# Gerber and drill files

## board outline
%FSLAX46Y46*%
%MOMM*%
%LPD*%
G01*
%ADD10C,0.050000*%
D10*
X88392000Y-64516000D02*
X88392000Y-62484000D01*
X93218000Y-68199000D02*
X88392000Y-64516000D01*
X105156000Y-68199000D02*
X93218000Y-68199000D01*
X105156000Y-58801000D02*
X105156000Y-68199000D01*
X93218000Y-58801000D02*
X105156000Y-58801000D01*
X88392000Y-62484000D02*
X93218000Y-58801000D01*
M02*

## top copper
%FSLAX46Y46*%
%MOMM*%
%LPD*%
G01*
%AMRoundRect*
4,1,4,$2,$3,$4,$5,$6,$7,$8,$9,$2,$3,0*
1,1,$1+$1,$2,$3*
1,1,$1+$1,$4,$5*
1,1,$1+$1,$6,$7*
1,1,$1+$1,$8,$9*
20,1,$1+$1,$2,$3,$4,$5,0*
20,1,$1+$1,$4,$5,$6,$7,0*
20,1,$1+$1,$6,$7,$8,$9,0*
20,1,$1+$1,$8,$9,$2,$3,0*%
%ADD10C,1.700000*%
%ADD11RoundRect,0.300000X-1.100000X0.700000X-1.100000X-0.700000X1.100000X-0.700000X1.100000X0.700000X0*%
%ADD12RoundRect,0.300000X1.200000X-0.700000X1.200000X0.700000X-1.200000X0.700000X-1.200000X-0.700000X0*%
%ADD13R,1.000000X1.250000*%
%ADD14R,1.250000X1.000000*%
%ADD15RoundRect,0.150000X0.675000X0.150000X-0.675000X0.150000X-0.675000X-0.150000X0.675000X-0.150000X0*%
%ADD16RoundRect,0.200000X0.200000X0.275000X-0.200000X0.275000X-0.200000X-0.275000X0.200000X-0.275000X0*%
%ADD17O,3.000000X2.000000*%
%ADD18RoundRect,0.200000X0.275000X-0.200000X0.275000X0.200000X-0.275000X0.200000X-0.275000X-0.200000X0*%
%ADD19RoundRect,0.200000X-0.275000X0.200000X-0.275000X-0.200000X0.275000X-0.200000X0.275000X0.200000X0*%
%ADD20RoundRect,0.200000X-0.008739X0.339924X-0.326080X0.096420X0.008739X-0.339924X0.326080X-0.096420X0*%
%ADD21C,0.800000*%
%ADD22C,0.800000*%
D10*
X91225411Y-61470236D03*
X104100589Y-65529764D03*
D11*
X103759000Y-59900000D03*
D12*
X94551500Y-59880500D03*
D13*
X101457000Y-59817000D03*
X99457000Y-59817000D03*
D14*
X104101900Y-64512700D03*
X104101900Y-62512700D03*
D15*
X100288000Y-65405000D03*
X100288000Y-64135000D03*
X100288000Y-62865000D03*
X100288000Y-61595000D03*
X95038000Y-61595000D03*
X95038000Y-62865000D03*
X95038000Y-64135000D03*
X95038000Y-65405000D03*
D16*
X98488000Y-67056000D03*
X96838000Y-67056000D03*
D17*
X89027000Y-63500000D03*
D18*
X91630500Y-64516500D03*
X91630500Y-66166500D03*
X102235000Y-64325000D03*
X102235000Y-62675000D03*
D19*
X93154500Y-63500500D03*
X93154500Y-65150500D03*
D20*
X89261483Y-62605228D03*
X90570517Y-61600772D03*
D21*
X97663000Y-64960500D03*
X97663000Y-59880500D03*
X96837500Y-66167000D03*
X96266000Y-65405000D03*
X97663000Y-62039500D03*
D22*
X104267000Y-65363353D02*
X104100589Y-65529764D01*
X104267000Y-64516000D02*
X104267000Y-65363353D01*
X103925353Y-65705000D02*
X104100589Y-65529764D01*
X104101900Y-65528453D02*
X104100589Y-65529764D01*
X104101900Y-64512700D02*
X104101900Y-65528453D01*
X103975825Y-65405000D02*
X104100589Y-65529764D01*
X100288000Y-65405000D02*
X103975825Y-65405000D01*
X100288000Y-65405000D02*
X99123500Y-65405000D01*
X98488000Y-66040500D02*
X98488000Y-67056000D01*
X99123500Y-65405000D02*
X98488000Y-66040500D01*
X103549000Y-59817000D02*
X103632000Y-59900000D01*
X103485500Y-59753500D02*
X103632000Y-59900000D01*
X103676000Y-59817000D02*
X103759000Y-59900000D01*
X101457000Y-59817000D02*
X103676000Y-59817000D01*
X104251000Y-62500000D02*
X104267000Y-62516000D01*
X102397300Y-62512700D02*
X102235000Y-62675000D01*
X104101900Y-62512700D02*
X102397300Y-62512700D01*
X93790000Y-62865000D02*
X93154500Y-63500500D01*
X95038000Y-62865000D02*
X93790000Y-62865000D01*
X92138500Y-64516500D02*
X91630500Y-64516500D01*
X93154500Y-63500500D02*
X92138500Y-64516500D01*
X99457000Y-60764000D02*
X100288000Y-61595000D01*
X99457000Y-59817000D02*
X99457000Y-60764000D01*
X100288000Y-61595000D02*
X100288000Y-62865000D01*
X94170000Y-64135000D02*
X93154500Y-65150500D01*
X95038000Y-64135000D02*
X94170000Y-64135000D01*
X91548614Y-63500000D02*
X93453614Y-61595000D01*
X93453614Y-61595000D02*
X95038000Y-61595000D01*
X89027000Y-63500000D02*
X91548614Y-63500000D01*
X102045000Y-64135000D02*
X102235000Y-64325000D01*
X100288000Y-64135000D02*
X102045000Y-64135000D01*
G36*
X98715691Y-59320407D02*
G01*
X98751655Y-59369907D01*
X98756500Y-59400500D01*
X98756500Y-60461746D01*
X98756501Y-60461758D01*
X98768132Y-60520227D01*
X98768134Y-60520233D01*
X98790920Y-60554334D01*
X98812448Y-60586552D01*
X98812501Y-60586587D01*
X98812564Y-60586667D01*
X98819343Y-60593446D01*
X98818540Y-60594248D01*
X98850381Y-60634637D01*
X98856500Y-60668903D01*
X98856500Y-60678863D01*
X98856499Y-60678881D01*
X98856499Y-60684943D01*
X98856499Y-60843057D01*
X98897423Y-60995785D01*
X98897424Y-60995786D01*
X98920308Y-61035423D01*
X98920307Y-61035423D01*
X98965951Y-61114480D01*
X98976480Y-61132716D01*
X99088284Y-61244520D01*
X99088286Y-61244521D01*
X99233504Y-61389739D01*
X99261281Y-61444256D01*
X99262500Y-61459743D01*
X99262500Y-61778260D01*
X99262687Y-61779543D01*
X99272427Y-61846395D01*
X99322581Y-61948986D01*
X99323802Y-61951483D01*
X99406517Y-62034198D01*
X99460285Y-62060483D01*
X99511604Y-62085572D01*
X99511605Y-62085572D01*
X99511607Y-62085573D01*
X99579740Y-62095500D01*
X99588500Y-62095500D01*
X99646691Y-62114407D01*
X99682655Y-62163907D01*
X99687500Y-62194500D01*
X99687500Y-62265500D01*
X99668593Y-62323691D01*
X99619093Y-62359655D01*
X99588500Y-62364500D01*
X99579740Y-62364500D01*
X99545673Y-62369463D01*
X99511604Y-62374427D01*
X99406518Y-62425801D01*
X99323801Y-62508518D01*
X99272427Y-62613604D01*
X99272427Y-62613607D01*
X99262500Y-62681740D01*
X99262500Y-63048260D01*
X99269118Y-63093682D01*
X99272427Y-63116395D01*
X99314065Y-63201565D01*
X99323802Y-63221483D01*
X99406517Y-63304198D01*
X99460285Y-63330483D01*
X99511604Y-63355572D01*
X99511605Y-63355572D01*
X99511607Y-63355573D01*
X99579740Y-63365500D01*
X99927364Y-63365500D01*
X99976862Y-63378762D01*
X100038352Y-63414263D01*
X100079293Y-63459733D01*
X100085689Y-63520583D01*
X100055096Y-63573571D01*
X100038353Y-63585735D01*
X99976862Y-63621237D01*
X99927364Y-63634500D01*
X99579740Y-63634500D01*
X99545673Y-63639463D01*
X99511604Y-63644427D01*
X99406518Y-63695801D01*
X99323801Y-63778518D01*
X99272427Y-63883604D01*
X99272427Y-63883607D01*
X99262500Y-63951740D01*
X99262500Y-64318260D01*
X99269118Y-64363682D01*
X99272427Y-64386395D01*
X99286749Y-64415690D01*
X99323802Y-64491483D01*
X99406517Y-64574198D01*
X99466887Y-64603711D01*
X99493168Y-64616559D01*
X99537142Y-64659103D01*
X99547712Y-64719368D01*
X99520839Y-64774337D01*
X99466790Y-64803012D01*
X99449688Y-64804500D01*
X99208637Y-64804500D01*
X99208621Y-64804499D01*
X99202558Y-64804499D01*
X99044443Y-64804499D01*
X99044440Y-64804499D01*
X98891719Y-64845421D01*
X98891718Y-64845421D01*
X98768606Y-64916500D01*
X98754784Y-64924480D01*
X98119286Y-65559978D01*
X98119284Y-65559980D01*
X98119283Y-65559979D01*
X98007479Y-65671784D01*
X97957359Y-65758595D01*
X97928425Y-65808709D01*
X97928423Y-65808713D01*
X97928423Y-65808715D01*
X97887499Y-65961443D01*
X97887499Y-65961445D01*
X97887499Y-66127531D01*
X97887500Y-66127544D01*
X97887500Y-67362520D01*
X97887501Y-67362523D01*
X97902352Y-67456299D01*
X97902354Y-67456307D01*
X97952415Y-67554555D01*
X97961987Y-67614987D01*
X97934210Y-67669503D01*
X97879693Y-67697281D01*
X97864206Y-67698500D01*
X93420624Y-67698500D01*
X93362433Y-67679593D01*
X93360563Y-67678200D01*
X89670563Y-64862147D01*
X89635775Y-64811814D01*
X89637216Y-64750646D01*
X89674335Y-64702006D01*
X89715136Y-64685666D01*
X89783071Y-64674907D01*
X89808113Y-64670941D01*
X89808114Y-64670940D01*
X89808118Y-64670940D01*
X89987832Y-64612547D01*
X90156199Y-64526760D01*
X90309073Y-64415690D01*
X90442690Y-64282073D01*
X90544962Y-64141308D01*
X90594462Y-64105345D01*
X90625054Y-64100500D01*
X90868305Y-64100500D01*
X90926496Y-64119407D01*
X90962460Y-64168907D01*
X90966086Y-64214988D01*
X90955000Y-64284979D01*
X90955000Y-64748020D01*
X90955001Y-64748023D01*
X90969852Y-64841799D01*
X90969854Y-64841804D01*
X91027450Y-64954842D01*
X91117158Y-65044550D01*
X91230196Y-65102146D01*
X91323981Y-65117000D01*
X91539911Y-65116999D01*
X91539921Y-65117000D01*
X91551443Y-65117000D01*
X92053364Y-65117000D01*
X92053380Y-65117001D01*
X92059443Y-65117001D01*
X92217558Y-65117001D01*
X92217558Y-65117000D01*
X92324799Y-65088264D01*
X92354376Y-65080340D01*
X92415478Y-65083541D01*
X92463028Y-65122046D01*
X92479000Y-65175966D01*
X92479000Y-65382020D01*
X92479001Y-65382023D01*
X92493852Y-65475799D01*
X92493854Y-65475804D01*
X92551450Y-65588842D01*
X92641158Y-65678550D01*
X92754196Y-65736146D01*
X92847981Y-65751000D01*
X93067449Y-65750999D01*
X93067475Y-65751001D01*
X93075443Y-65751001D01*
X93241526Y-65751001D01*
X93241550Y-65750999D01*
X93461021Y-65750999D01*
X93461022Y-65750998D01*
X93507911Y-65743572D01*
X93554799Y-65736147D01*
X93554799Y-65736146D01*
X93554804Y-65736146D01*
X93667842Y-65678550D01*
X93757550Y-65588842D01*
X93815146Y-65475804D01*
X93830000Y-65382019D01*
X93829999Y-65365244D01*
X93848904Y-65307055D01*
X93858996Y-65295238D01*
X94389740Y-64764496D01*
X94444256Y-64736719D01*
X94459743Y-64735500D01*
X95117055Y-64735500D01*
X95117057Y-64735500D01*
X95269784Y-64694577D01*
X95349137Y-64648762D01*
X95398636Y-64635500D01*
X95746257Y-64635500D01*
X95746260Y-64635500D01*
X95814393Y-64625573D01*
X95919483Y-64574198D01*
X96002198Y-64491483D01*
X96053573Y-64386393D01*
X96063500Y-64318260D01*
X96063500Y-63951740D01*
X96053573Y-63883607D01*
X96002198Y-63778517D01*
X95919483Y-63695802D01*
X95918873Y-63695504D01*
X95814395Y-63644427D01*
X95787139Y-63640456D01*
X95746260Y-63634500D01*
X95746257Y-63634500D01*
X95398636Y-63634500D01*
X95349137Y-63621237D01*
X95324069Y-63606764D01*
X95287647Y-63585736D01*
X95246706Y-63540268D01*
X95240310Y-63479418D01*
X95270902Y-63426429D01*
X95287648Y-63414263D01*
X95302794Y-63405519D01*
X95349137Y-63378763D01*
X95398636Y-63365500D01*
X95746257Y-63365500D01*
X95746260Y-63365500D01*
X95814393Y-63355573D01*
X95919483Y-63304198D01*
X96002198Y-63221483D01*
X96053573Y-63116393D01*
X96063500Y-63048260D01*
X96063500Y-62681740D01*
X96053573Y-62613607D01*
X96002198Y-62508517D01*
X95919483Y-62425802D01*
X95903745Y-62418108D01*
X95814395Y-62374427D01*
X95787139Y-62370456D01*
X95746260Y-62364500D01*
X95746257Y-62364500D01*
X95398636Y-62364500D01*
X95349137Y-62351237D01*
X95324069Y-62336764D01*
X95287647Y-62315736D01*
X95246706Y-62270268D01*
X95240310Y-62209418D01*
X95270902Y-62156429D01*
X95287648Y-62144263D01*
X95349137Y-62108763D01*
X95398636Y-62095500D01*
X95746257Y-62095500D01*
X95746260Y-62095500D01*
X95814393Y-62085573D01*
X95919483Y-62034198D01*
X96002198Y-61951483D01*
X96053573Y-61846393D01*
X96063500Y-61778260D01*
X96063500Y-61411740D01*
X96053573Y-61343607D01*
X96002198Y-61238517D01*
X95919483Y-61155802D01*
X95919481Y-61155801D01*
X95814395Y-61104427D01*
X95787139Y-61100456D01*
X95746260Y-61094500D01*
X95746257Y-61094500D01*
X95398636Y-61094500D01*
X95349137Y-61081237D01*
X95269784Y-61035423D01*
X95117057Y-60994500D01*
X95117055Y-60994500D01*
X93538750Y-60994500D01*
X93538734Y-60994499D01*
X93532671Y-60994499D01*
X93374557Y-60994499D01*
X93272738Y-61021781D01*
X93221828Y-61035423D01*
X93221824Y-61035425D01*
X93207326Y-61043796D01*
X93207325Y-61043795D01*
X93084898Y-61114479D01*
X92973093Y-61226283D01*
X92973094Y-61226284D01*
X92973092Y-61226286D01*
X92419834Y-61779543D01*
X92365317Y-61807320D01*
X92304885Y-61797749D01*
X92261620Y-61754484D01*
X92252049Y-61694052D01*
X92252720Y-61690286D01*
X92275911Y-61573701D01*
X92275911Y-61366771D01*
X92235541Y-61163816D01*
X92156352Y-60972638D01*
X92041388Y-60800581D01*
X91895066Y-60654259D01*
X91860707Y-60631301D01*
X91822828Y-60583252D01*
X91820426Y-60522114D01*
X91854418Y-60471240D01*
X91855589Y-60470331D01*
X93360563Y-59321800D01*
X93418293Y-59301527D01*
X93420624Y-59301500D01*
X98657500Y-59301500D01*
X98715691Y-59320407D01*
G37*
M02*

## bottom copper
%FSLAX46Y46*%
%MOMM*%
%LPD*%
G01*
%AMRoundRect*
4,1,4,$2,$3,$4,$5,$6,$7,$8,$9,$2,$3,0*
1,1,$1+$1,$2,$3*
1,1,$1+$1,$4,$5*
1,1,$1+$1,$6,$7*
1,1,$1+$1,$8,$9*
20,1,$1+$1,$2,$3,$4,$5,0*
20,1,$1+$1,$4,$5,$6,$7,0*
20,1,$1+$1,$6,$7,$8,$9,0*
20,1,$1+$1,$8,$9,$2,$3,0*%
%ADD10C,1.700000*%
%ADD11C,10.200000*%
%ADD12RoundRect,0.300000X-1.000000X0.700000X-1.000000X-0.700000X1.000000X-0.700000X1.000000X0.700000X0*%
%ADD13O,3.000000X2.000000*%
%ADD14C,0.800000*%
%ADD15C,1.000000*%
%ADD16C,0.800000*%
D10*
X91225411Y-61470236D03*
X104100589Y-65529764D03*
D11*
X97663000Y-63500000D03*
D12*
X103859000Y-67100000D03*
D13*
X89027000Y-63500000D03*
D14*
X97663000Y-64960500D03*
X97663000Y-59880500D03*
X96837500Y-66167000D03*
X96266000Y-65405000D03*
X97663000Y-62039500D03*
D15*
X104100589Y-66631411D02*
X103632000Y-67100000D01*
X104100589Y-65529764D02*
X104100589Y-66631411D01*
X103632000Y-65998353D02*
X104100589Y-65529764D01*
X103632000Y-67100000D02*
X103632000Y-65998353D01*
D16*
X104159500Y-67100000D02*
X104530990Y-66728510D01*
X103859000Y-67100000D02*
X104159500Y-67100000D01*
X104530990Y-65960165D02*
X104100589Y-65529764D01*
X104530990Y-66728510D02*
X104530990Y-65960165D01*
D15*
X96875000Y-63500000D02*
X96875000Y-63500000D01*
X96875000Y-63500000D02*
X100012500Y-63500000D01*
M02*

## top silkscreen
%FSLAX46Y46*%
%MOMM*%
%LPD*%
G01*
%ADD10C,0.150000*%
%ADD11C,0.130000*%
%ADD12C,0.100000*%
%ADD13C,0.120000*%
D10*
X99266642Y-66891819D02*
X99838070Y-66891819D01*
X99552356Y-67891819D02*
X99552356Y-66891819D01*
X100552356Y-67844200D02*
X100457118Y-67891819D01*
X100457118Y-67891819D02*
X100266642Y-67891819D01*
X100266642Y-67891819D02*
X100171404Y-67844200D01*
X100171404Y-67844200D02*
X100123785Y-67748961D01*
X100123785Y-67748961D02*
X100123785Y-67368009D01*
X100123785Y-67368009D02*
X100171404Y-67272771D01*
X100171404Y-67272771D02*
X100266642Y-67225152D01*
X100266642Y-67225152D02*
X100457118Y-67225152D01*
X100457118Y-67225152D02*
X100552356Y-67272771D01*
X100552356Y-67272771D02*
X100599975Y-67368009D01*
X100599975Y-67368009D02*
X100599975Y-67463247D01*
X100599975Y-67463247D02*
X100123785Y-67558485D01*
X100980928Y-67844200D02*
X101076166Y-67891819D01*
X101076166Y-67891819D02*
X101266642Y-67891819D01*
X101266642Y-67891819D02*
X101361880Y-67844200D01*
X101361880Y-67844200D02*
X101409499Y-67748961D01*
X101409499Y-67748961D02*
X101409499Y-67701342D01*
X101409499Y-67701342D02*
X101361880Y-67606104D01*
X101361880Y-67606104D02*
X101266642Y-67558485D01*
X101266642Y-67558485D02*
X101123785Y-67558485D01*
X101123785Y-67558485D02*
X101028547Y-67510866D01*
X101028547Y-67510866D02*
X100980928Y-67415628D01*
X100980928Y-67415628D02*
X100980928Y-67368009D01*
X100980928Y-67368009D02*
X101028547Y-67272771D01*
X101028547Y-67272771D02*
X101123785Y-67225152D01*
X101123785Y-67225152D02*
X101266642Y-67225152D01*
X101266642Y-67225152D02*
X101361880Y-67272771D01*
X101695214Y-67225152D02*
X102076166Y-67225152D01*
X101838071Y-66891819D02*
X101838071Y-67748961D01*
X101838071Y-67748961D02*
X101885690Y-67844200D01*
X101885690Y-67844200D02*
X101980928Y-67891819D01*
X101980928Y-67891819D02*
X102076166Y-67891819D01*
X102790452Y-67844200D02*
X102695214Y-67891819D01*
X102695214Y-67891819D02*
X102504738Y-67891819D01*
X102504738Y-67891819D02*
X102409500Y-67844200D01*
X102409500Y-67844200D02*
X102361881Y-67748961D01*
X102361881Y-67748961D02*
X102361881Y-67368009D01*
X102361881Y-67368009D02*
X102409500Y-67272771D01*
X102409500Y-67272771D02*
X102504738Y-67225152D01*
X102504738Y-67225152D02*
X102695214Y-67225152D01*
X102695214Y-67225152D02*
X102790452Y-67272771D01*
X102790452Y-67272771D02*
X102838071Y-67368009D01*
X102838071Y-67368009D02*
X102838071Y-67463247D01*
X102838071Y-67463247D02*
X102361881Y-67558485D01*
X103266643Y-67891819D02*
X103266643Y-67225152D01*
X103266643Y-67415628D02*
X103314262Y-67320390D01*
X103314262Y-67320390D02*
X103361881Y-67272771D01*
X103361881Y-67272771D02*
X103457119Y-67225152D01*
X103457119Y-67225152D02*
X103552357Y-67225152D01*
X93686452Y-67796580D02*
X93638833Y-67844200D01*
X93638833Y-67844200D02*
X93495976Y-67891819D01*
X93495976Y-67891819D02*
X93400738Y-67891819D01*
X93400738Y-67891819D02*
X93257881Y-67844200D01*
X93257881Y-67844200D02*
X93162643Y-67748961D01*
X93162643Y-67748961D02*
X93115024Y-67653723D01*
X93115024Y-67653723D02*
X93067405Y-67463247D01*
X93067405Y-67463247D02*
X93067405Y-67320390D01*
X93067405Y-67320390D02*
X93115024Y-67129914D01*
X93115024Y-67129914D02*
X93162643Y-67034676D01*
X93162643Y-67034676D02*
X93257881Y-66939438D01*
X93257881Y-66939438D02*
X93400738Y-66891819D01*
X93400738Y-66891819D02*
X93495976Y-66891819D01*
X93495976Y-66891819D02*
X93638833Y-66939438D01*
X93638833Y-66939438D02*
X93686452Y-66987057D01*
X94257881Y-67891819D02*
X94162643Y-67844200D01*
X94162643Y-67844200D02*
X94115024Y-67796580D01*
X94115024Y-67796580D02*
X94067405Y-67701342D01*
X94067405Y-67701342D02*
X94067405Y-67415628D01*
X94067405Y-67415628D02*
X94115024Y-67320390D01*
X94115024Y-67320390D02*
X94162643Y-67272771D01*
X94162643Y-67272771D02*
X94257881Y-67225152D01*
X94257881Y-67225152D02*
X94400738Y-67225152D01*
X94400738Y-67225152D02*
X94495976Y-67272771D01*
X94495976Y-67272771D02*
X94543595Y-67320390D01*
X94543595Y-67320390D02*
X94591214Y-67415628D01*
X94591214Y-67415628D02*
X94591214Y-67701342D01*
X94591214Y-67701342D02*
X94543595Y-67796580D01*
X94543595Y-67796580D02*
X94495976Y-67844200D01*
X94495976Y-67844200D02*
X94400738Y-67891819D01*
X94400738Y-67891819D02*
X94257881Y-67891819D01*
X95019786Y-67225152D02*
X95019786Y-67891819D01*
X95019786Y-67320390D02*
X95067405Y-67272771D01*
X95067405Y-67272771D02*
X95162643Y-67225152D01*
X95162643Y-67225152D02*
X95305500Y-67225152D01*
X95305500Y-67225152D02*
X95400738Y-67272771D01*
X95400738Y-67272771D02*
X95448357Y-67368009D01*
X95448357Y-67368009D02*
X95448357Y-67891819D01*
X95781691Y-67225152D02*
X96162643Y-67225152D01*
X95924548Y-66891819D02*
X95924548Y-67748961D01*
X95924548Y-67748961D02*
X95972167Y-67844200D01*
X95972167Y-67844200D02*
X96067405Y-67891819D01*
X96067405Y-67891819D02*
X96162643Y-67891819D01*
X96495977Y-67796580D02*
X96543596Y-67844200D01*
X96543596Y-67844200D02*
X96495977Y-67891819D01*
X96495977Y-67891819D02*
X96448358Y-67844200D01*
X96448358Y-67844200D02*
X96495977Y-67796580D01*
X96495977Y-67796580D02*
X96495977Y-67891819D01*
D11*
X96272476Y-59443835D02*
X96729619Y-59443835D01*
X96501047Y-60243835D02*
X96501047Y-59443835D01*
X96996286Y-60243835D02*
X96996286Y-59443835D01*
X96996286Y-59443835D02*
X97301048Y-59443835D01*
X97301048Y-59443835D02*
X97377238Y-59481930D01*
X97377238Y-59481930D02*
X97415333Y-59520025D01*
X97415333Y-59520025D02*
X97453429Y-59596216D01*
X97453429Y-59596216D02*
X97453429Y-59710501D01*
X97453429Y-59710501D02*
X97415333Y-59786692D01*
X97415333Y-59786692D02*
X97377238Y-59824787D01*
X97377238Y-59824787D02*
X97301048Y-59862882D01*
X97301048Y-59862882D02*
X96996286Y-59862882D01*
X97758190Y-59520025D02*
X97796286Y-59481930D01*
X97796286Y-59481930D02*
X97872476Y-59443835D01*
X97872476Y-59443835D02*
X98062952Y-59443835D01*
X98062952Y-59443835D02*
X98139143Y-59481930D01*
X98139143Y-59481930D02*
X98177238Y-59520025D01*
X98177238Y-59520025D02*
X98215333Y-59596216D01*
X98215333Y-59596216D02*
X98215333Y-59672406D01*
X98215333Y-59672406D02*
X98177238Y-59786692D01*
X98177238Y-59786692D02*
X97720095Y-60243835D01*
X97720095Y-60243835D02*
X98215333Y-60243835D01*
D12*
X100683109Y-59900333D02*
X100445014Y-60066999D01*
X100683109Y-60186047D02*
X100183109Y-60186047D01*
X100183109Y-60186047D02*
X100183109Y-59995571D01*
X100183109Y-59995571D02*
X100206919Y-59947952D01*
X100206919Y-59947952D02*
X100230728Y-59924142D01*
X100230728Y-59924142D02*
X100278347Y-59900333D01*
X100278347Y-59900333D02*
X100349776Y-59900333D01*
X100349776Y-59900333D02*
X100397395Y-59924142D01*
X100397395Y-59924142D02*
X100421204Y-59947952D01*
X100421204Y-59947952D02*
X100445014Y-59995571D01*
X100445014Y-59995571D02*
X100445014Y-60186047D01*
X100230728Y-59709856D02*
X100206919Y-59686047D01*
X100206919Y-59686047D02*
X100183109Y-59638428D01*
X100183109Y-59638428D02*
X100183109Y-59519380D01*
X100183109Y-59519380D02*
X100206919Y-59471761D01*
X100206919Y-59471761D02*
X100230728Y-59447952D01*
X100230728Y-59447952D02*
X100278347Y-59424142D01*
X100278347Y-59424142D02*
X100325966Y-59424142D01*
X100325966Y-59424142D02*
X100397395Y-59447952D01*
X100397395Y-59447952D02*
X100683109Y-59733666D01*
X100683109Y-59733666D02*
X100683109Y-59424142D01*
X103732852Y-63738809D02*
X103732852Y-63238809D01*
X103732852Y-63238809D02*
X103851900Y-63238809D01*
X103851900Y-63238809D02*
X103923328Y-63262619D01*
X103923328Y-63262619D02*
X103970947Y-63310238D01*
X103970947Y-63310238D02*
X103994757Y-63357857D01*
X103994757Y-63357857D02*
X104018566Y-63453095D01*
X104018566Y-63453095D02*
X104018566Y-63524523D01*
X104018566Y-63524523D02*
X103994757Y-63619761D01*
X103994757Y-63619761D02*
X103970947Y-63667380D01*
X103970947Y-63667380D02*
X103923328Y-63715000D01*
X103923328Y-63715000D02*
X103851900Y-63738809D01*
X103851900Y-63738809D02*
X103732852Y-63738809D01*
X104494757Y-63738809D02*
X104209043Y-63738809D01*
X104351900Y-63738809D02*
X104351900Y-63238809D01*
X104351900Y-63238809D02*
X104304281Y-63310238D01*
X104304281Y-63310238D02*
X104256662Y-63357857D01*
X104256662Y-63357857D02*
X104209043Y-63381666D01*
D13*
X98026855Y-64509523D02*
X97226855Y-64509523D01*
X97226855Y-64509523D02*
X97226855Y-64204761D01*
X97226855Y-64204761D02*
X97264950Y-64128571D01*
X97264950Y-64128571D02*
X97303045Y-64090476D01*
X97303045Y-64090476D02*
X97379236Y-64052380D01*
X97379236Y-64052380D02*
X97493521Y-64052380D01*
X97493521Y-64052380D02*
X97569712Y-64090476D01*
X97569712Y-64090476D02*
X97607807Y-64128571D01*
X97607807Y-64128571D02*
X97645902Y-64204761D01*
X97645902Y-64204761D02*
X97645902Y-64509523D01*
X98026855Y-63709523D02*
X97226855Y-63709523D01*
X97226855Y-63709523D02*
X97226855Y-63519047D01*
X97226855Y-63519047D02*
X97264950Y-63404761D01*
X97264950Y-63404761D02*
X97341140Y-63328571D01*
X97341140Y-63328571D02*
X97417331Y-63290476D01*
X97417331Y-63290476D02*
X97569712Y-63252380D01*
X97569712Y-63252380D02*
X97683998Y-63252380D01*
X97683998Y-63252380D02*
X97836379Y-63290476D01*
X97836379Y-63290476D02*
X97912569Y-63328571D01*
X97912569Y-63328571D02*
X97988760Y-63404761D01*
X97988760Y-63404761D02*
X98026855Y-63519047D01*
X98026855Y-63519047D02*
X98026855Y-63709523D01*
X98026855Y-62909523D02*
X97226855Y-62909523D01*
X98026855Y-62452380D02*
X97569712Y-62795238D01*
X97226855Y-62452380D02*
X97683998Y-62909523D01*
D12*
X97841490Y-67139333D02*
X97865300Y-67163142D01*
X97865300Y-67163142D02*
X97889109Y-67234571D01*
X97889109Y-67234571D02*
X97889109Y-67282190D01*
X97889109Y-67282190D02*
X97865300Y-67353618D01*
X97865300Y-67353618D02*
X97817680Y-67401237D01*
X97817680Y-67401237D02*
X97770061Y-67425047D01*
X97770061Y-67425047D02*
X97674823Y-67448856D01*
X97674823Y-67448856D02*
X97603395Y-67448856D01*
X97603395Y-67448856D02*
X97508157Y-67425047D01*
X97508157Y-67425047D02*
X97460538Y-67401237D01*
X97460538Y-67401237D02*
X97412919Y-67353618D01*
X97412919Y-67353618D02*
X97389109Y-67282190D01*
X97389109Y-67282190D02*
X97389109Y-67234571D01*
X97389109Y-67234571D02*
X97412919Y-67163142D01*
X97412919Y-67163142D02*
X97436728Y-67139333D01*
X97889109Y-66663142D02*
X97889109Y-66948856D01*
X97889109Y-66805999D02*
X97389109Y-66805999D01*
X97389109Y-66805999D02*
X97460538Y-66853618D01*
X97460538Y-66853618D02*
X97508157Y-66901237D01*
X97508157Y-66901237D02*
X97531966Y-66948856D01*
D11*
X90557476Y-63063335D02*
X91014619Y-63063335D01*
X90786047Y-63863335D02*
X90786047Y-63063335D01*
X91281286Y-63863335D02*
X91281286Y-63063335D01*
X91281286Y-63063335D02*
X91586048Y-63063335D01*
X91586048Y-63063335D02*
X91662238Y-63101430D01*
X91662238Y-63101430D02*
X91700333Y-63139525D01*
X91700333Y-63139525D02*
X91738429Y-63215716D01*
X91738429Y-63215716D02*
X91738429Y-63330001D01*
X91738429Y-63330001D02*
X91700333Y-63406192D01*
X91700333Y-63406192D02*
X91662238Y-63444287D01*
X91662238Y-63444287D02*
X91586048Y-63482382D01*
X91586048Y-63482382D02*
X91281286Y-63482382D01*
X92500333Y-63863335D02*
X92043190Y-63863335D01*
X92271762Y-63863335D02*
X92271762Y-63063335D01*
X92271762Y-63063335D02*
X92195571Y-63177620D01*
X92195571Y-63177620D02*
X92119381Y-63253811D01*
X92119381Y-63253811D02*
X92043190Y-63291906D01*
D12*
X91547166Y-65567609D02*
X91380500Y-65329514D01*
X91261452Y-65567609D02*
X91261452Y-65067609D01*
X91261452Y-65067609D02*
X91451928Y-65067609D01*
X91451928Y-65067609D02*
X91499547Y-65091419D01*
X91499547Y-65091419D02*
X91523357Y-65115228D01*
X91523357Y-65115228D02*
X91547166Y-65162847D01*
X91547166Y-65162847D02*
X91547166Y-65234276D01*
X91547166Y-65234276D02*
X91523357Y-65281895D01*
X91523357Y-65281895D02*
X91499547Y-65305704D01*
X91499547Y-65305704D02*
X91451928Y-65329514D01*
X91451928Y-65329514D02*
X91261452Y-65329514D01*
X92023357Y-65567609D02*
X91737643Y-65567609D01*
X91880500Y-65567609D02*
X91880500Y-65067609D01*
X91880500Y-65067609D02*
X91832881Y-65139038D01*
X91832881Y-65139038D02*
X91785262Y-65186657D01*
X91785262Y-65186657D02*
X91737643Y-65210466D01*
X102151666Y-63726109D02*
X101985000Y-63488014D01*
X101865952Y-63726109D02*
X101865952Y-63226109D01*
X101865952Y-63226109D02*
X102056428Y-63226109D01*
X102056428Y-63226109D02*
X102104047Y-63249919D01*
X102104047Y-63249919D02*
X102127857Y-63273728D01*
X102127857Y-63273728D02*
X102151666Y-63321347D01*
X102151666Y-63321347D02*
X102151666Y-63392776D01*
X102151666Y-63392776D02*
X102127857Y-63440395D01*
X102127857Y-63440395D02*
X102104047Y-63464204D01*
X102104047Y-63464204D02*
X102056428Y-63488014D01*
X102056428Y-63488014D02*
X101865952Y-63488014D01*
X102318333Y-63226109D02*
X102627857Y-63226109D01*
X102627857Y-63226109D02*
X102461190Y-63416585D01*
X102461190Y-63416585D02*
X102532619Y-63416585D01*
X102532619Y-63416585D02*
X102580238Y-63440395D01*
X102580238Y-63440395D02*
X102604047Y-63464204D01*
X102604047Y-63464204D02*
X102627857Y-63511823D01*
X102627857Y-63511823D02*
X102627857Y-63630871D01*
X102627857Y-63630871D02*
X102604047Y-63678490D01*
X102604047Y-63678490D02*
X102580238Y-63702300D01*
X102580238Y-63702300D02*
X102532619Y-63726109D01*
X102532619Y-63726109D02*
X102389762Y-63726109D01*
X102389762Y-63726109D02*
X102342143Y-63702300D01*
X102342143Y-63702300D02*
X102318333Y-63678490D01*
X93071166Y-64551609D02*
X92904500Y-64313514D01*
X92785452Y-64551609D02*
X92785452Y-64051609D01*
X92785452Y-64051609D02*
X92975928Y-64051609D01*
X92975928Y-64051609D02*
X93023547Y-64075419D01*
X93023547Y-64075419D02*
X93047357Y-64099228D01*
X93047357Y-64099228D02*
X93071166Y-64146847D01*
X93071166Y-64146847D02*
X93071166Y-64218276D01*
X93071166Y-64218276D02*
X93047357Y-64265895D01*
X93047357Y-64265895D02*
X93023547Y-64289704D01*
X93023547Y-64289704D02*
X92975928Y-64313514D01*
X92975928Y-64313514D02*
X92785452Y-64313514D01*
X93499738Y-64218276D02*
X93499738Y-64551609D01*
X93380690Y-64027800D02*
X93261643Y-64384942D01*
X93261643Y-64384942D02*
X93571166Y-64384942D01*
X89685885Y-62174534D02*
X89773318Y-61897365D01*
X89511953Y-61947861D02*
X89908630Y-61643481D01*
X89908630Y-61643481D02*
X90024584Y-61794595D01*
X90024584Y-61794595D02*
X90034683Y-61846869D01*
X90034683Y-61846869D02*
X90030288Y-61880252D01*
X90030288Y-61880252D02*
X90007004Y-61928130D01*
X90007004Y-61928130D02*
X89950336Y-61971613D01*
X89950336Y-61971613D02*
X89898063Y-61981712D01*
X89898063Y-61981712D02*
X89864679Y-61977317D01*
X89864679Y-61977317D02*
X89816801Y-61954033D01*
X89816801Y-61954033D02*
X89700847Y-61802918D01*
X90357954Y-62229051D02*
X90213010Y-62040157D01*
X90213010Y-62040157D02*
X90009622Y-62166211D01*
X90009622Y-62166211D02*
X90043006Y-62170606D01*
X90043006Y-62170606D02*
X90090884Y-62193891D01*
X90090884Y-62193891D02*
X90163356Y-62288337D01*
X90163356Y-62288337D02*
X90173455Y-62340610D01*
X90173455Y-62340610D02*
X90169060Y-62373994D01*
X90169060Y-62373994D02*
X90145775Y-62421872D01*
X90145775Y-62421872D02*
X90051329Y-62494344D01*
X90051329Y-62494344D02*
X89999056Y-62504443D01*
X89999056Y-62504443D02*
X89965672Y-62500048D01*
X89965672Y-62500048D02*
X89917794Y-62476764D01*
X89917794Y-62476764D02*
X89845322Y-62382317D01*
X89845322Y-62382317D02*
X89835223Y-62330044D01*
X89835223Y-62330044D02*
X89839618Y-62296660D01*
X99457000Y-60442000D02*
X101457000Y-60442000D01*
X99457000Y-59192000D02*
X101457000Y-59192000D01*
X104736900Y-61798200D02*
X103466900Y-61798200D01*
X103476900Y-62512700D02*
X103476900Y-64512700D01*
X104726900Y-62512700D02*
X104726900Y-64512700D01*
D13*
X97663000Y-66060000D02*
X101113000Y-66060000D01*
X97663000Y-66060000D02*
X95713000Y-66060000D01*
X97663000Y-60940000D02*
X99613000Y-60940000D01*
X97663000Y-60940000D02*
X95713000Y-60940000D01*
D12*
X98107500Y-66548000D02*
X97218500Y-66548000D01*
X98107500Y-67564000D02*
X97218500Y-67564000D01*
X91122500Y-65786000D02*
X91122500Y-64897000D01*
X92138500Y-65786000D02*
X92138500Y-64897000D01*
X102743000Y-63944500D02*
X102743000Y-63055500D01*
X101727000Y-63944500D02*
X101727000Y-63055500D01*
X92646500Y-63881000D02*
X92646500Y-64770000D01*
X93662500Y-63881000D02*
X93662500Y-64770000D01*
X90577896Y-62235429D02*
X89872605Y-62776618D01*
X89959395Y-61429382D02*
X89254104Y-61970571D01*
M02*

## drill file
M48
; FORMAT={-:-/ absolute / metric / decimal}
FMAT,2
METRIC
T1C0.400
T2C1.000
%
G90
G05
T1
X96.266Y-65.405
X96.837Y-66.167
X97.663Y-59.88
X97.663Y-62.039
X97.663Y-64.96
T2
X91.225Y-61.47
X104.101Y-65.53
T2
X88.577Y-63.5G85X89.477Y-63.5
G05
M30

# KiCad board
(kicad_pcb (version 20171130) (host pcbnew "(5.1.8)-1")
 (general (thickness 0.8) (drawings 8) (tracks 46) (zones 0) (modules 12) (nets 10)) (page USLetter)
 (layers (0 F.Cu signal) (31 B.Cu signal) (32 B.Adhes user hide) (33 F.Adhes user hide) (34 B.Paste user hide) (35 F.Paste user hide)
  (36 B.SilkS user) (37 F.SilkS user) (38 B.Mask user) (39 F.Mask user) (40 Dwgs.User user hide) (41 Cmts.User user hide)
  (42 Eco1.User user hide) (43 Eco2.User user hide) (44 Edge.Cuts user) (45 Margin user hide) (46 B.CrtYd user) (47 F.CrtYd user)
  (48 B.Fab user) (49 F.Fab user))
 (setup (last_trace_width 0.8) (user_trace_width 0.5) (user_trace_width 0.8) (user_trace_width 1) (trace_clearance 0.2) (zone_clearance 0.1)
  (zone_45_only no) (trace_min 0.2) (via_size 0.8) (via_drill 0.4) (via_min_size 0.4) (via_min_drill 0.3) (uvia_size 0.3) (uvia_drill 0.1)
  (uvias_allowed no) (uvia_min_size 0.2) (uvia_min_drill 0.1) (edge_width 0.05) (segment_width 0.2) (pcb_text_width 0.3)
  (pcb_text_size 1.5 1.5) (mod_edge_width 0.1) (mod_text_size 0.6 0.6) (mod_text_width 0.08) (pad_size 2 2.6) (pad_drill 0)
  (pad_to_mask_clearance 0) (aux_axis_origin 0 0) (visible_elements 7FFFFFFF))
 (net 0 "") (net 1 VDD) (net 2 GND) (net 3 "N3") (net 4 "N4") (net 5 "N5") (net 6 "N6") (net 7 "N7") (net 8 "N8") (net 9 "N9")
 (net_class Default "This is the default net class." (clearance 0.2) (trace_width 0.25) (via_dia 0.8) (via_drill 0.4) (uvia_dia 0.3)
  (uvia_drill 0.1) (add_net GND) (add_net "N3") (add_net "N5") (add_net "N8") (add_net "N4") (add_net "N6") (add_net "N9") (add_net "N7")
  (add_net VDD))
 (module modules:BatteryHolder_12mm (layer B.Cu) (at 97.663 63.5 342.5)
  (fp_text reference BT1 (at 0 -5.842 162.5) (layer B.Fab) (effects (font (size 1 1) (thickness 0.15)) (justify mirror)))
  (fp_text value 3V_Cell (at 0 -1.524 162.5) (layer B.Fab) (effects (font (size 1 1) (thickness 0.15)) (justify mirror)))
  (pad 1 thru_hole circle (at -6.75 0 342.5) (size 1.7 1.7) (drill 1) (layers *.Cu *.Mask) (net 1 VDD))
  (pad 1 thru_hole circle (at 6.75 0 342.5) (size 1.7 1.7) (drill 1) (layers *.Cu *.Mask) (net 1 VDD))
  (pad 2 smd circle (at 0 0 342.5) (size 10.2 10.2) (layers B.Cu B.Mask) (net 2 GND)))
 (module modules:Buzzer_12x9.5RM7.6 (layer F.Cu) (at 103.759 63.5 270)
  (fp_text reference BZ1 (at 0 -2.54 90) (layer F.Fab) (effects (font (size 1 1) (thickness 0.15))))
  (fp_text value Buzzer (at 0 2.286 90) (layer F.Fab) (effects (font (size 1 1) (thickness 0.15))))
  (pad 2 smd roundrect (at -3.6 0 270) (size 2 2.8) (layers F.Cu F.Paste F.Mask) (roundrect_rratio 0.15) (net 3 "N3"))
  (pad 1 smd roundrect (at 3.6 -0.1 270) (size 2 2.6) (layers B.Cu B.Paste B.Mask) (roundrect_rratio 0.15) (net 1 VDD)))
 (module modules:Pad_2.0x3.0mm (layer F.Cu) (at 94.5515 59.8805 90)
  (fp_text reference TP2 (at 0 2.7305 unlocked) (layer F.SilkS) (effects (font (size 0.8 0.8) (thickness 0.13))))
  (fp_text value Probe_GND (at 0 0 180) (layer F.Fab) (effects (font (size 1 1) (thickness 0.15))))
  (pad 1 smd roundrect (at 0 0 90) (size 2 3) (layers F.Cu F.Mask) (roundrect_rratio 0.15) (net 2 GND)))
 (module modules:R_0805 (layer F.Cu) (at 100.457 59.817)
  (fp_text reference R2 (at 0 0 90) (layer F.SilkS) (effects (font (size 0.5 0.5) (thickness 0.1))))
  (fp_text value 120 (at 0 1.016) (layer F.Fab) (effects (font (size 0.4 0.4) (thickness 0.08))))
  (fp_line (start -1 0.625) (end 1 0.625) (layer F.SilkS) (width 0.1))
  (fp_line (start -1 -0.625) (end 1 -0.625) (layer F.SilkS) (width 0.1))
  (pad 2 smd rect (at 1 0) (size 1 1.25) (layers F.Cu F.Paste F.Mask) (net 3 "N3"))
  (pad 1 smd rect (at -1 0) (size 1 1.25) (layers F.Cu F.Paste F.Mask) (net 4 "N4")))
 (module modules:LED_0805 (layer F.Cu) (at 104.1019 63.5127 270)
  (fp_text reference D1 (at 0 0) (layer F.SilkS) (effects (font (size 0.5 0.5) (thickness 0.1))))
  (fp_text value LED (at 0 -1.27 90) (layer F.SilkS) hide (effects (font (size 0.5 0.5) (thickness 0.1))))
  (fp_line (start -1.7145 -0.635) (end -1.7145 0.635) (layer F.SilkS) (width 0.1))
  (fp_line (start -1 0.625) (end 1 0.625) (layer F.SilkS) (width 0.1))
  (fp_line (start -1 -0.625) (end 1 -0.625) (layer F.SilkS) (width 0.1))
  (pad 2 smd rect (at 1 0 270) (size 1 1.25) (layers F.Cu F.Paste F.Mask) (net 1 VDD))
  (pad 1 smd rect (at -1 0 270) (size 1 1.25) (layers F.Cu F.Paste F.Mask) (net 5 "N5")))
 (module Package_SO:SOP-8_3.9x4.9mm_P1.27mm (layer F.Cu) (at 97.663 63.5 180)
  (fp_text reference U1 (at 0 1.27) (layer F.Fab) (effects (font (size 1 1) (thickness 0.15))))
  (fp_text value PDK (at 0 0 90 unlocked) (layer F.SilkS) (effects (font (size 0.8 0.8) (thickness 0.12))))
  (fp_line (start 0 -2.56) (end -3.45 -2.56) (layer F.SilkS) (width 0.12))
  (fp_line (start 0 -2.56) (end 1.95 -2.56) (layer F.SilkS) (width 0.12))
  (fp_line (start 0 2.56) (end -1.95 2.56) (layer F.SilkS) (width 0.12))
  (fp_line (start 0 2.56) (end 1.95 2.56) (layer F.SilkS) (width 0.12))
  (pad 1 smd roundrect (at -2.625 -1.905 180) (size 1.65 0.6) (layers F.Cu F.Paste F.Mask) (roundrect_rratio 0.25) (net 1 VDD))
  (pad 2 smd roundrect (at -2.625 -0.635 180) (size 1.65 0.6) (layers F.Cu F.Paste F.Mask) (roundrect_rratio 0.25) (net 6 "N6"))
  (pad 3 smd roundrect (at -2.625 0.635 180) (size 1.65 0.6) (layers F.Cu F.Paste F.Mask) (roundrect_rratio 0.25) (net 4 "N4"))
  (pad 4 smd roundrect (at -2.625 1.905 180) (size 1.65 0.6) (layers F.Cu F.Paste F.Mask) (roundrect_rratio 0.25) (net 4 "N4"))
  (pad 5 smd roundrect (at 2.625 1.905 180) (size 1.65 0.6) (layers F.Cu F.Paste F.Mask) (roundrect_rratio 0.25) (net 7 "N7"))
  (pad 6 smd roundrect (at 2.625 0.635 180) (size 1.65 0.6) (layers F.Cu F.Paste F.Mask) (roundrect_rratio 0.25) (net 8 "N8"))
  (pad 7 smd roundrect (at 2.625 -0.635 180) (size 1.65 0.6) (layers F.Cu F.Paste F.Mask) (roundrect_rratio 0.25) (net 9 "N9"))
  (pad 8 smd roundrect (at 2.625 -1.905 180) (size 1.65 0.6) (layers F.Cu F.Paste F.Mask) (roundrect_rratio 0.25) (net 2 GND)))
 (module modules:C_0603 (layer F.Cu) (at 97.663 67.056 180)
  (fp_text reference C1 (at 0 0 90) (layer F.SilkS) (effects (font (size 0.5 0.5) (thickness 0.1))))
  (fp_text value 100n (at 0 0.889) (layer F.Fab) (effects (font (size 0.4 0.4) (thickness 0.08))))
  (fp_line (start -0.4445 0.508) (end 0.4445 0.508) (layer F.SilkS) (width 0.1))
  (fp_line (start -0.4445 -0.508) (end 0.4445 -0.508) (layer F.SilkS) (width 0.1))
  (pad 1 smd roundrect (at -0.825 0 180) (size 0.8 0.95) (layers F.Cu F.Paste F.Mask) (roundrect_rratio 0.25) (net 1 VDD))
  (pad 2 smd roundrect (at 0.825 0 180) (size 0.8 0.95) (layers F.Cu F.Paste F.Mask) (roundrect_rratio 0.25) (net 2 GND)))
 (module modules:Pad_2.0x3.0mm (layer F.Cu) (at 89.027 63.5 90)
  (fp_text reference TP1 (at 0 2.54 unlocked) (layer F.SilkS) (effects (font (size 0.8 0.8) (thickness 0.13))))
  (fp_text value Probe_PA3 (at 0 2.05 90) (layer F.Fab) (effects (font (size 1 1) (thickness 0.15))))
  (pad 1 thru_hole oval (at 0 0 90) (size 2 3) (drill oval 1 1.9) (layers *.Cu *.Mask) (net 7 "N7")))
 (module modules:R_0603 (layer F.Cu) (at 91.6305 65.3415 90)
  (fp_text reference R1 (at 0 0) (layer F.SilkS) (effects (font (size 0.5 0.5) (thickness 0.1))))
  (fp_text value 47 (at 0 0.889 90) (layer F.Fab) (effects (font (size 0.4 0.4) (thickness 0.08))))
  (fp_line (start -0.4445 -0.508) (end 0.4445 -0.508) (layer F.SilkS) (width 0.1))
  (fp_line (start -0.4445 0.508) (end 0.4445 0.508) (layer F.SilkS) (width 0.1))
  (pad 2 smd roundrect (at 0.825 0 90) (size 0.8 0.95) (layers F.Cu F.Paste F.Mask) (roundrect_rratio 0.25) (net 8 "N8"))
  (pad 1 smd roundrect (at -0.825 0 90) (size 0.8 0.95) (layers F.Cu F.Paste F.Mask) (roundrect_rratio 0.25) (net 2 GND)))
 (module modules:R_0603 (layer F.Cu) (at 102.235 63.5 90)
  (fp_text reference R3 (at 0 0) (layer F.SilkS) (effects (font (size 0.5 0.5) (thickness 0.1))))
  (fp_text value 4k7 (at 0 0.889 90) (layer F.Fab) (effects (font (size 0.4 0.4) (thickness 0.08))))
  (fp_line (start -0.4445 0.508) (end 0.4445 0.508) (layer F.SilkS) (width 0.1))
  (fp_line (start -0.4445 -0.508) (end 0.4445 -0.508) (layer F.SilkS) (width 0.1))
  (pad 1 smd roundrect (at -0.825 0 90) (size 0.8 0.95) (layers F.Cu F.Paste F.Mask) (roundrect_rratio 0.25) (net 6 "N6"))
  (pad 2 smd roundrect (at 0.825 0 90) (size 0.8 0.95) (layers F.Cu F.Paste F.Mask) (roundrect_rratio 0.25) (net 5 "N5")))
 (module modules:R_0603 (layer F.Cu) (at 93.1545 64.3255 270)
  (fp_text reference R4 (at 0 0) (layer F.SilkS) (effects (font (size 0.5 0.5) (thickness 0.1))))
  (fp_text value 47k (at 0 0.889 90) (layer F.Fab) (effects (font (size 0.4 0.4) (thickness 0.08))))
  (fp_line (start -0.4445 0.508) (end 0.4445 0.508) (layer F.SilkS) (width 0.1))
  (fp_line (start -0.4445 -0.508) (end 0.4445 -0.508) (layer F.SilkS) (width 0.1))
  (pad 1 smd roundrect (at -0.825 0 270) (size 0.8 0.95) (layers F.Cu F.Paste F.Mask) (roundrect_rratio 0.25) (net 8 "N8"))
  (pad 2 smd roundrect (at 0.825 0 270) (size 0.8 0.95) (layers F.Cu F.Paste F.Mask) (roundrect_rratio 0.25) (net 9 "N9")))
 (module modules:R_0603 (layer F.Cu) (at 89.916 62.103 217.5)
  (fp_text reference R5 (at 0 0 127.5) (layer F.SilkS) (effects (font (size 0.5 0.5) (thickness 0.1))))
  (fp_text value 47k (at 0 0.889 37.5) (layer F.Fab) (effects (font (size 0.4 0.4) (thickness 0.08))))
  (fp_line (start -0.4445 -0.508) (end 0.4445 -0.508) (layer F.SilkS) (width 0.1))
  (fp_line (start -0.4445 0.508) (end 0.4445 0.508) (layer F.SilkS) (width 0.1))
  (pad 2 smd roundrect (at 0.825 0 217.5) (size 0.8 0.95) (layers F.Cu F.Paste F.Mask) (roundrect_rratio 0.25) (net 7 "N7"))
  (pad 1 smd roundrect (at -0.825 0 217.5) (size 0.8 0.95) (layers F.Cu F.Paste F.Mask) (roundrect_rratio 0.25) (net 1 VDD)))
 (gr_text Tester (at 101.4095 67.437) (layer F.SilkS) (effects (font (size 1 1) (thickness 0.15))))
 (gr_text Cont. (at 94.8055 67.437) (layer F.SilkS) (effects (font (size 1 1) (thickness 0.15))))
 (gr_line (start 88.392 64.516) (end 88.392 62.484) (layer Edge.Cuts) (width 0.05))
 (gr_line (start 93.218 68.199) (end 88.392 64.516) (layer Edge.Cuts) (width 0.05))
 (gr_line (start 105.156 68.199) (end 93.218 68.199) (layer Edge.Cuts) (width 0.05))
 (gr_line (start 105.156 58.801) (end 105.156 68.199) (layer Edge.Cuts) (width 0.05))
 (gr_line (start 93.218 58.801) (end 105.156 58.801) (layer Edge.Cuts) (width 0.05))
 (gr_line (start 88.392 62.484) (end 93.218 58.801) (layer Edge.Cuts) (width 0.05))
 (segment (start 104.267 65.363353) (end 104.100589 65.529764) (width 0.8) (layer F.Cu) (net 1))
 (segment (start 104.267 64.516) (end 104.267 65.363353) (width 0.8) (layer F.Cu) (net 1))
 (segment (start 103.925353 65.705) (end 104.100589 65.529764) (width 0.8) (layer F.Cu) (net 1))
 (segment (start 104.100589 66.631411) (end 103.632 67.1) (width 1) (layer B.Cu) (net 1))
 (segment (start 104.100589 65.529764) (end 104.100589 66.631411) (width 1) (layer B.Cu) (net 1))
 (segment (start 103.632 65.998353) (end 104.100589 65.529764) (width 1) (layer B.Cu) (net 1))
 (segment (start 103.632 67.1) (end 103.632 65.998353) (width 1) (layer B.Cu) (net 1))
 (segment (start 104.1019 65.528453) (end 104.100589 65.529764) (width 0.8) (layer F.Cu) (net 1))
 (segment (start 104.1019 64.5127) (end 104.1019 65.528453) (width 0.8) (layer F.Cu) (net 1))
 (segment (start 103.975825 65.405) (end 104.100589 65.529764) (width 0.8) (layer F.Cu) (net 1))
 (segment (start 100.288 65.405) (end 103.975825 65.405) (width 0.8) (layer F.Cu) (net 1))
 (segment (start 100.288 65.405) (end 99.1235 65.405) (width 0.8) (layer F.Cu) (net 1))
 (segment (start 98.488 66.0405) (end 98.488 67.056) (width 0.8) (layer F.Cu) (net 1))
 (segment (start 99.1235 65.405) (end 98.488 66.0405) (width 0.8) (layer F.Cu) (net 1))
 (segment (start 104.1595 67.1) (end 104.53099 66.72851) (width 0.8) (layer B.Cu) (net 1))
 (segment (start 103.859 67.1) (end 104.1595 67.1) (width 0.8) (layer B.Cu) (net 1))
 (segment (start 104.53099 65.960165) (end 104.100589 65.529764) (width 0.8) (layer B.Cu) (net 1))
 (segment (start 104.53099 66.72851) (end 104.53099 65.960165) (width 0.8) (layer B.Cu) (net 1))
 (segment (start 103.549 59.817) (end 103.632 59.9) (width 0.8) (layer F.Cu) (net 3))
 (segment (start 103.4855 59.7535) (end 103.632 59.9) (width 0.8) (layer F.Cu) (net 3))
 (segment (start 103.676 59.817) (end 103.759 59.9) (width 0.8) (layer F.Cu) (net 3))
 (segment (start 101.457 59.817) (end 103.676 59.817) (width 0.8) (layer F.Cu) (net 3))
 (segment (start 104.251 62.5) (end 104.267 62.516) (width 0.8) (layer F.Cu) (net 5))
 (segment (start 102.3973 62.5127) (end 102.235 62.675) (width 0.8) (layer F.Cu) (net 5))
 (segment (start 104.1019 62.5127) (end 102.3973 62.5127) (width 0.8) (layer F.Cu) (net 5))
 (via (at 97.663 64.9605) (size 0.8) (drill 0.4) (layers F.Cu B.Cu) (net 2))
 (via (at 97.663 59.8805) (size 0.8) (drill 0.4) (layers F.Cu B.Cu) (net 2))
 (via (at 96.8375 66.167) (size 0.8) (drill 0.4) (layers F.Cu B.Cu) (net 2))
 (via (at 96.266 65.405) (size 0.8) (drill 0.4) (layers F.Cu B.Cu) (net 2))
 (segment (start 96.875 63.5) (end 96.875 63.5) (width 1) (layer B.Cu) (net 2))
 (segment (start 96.875 63.5) (end 100.0125 63.5) (width 1) (layer B.Cu) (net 2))
 (via (at 97.663 62.0395) (size 0.8) (drill 0.4) (layers F.Cu B.Cu) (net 2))
 (segment (start 93.79 62.865) (end 93.1545 63.5005) (width 0.8) (layer F.Cu) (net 8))
 (segment (start 95.038 62.865) (end 93.79 62.865) (width 0.8) (layer F.Cu) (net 8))
 (segment (start 92.1385 64.5165) (end 91.6305 64.5165) (width 0.8) (layer F.Cu) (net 8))
 (segment (start 93.1545 63.5005) (end 92.1385 64.5165) (width 0.8) (layer F.Cu) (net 8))
 (segment (start 99.457 60.764) (end 100.288 61.595) (width 0.8) (layer F.Cu) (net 4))
 (segment (start 99.457 59.817) (end 99.457 60.764) (width 0.8) (layer F.Cu) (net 4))
 (segment (start 100.288 61.595) (end 100.288 62.865) (width 0.8) (layer F.Cu) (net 4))
 (segment (start 94.17 64.135) (end 93.1545 65.1505) (width 0.8) (layer F.Cu) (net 9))
 (segment (start 95.038 64.135) (end 94.17 64.135) (width 0.8) (layer F.Cu) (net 9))
 (segment (start 91.548614 63.5) (end 93.453614 61.595) (width 0.8) (layer F.Cu) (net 7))
 (segment (start 93.453614 61.595) (end 95.038 61.595) (width 0.8) (layer F.Cu) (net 7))
 (segment (start 89.027 63.5) (end 91.548614 63.5) (width 0.8) (layer F.Cu) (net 7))
 (segment (start 102.045 64.135) (end 102.235 64.325) (width 0.8) (layer F.Cu) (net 6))
 (segment (start 100.288 64.135) (end 102.045 64.135) (width 0.8) (layer F.Cu) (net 6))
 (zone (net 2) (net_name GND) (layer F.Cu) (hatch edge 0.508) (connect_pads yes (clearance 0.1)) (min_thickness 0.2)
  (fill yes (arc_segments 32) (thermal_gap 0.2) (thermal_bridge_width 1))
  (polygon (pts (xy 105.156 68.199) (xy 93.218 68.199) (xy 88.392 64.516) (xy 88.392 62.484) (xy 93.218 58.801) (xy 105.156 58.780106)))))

